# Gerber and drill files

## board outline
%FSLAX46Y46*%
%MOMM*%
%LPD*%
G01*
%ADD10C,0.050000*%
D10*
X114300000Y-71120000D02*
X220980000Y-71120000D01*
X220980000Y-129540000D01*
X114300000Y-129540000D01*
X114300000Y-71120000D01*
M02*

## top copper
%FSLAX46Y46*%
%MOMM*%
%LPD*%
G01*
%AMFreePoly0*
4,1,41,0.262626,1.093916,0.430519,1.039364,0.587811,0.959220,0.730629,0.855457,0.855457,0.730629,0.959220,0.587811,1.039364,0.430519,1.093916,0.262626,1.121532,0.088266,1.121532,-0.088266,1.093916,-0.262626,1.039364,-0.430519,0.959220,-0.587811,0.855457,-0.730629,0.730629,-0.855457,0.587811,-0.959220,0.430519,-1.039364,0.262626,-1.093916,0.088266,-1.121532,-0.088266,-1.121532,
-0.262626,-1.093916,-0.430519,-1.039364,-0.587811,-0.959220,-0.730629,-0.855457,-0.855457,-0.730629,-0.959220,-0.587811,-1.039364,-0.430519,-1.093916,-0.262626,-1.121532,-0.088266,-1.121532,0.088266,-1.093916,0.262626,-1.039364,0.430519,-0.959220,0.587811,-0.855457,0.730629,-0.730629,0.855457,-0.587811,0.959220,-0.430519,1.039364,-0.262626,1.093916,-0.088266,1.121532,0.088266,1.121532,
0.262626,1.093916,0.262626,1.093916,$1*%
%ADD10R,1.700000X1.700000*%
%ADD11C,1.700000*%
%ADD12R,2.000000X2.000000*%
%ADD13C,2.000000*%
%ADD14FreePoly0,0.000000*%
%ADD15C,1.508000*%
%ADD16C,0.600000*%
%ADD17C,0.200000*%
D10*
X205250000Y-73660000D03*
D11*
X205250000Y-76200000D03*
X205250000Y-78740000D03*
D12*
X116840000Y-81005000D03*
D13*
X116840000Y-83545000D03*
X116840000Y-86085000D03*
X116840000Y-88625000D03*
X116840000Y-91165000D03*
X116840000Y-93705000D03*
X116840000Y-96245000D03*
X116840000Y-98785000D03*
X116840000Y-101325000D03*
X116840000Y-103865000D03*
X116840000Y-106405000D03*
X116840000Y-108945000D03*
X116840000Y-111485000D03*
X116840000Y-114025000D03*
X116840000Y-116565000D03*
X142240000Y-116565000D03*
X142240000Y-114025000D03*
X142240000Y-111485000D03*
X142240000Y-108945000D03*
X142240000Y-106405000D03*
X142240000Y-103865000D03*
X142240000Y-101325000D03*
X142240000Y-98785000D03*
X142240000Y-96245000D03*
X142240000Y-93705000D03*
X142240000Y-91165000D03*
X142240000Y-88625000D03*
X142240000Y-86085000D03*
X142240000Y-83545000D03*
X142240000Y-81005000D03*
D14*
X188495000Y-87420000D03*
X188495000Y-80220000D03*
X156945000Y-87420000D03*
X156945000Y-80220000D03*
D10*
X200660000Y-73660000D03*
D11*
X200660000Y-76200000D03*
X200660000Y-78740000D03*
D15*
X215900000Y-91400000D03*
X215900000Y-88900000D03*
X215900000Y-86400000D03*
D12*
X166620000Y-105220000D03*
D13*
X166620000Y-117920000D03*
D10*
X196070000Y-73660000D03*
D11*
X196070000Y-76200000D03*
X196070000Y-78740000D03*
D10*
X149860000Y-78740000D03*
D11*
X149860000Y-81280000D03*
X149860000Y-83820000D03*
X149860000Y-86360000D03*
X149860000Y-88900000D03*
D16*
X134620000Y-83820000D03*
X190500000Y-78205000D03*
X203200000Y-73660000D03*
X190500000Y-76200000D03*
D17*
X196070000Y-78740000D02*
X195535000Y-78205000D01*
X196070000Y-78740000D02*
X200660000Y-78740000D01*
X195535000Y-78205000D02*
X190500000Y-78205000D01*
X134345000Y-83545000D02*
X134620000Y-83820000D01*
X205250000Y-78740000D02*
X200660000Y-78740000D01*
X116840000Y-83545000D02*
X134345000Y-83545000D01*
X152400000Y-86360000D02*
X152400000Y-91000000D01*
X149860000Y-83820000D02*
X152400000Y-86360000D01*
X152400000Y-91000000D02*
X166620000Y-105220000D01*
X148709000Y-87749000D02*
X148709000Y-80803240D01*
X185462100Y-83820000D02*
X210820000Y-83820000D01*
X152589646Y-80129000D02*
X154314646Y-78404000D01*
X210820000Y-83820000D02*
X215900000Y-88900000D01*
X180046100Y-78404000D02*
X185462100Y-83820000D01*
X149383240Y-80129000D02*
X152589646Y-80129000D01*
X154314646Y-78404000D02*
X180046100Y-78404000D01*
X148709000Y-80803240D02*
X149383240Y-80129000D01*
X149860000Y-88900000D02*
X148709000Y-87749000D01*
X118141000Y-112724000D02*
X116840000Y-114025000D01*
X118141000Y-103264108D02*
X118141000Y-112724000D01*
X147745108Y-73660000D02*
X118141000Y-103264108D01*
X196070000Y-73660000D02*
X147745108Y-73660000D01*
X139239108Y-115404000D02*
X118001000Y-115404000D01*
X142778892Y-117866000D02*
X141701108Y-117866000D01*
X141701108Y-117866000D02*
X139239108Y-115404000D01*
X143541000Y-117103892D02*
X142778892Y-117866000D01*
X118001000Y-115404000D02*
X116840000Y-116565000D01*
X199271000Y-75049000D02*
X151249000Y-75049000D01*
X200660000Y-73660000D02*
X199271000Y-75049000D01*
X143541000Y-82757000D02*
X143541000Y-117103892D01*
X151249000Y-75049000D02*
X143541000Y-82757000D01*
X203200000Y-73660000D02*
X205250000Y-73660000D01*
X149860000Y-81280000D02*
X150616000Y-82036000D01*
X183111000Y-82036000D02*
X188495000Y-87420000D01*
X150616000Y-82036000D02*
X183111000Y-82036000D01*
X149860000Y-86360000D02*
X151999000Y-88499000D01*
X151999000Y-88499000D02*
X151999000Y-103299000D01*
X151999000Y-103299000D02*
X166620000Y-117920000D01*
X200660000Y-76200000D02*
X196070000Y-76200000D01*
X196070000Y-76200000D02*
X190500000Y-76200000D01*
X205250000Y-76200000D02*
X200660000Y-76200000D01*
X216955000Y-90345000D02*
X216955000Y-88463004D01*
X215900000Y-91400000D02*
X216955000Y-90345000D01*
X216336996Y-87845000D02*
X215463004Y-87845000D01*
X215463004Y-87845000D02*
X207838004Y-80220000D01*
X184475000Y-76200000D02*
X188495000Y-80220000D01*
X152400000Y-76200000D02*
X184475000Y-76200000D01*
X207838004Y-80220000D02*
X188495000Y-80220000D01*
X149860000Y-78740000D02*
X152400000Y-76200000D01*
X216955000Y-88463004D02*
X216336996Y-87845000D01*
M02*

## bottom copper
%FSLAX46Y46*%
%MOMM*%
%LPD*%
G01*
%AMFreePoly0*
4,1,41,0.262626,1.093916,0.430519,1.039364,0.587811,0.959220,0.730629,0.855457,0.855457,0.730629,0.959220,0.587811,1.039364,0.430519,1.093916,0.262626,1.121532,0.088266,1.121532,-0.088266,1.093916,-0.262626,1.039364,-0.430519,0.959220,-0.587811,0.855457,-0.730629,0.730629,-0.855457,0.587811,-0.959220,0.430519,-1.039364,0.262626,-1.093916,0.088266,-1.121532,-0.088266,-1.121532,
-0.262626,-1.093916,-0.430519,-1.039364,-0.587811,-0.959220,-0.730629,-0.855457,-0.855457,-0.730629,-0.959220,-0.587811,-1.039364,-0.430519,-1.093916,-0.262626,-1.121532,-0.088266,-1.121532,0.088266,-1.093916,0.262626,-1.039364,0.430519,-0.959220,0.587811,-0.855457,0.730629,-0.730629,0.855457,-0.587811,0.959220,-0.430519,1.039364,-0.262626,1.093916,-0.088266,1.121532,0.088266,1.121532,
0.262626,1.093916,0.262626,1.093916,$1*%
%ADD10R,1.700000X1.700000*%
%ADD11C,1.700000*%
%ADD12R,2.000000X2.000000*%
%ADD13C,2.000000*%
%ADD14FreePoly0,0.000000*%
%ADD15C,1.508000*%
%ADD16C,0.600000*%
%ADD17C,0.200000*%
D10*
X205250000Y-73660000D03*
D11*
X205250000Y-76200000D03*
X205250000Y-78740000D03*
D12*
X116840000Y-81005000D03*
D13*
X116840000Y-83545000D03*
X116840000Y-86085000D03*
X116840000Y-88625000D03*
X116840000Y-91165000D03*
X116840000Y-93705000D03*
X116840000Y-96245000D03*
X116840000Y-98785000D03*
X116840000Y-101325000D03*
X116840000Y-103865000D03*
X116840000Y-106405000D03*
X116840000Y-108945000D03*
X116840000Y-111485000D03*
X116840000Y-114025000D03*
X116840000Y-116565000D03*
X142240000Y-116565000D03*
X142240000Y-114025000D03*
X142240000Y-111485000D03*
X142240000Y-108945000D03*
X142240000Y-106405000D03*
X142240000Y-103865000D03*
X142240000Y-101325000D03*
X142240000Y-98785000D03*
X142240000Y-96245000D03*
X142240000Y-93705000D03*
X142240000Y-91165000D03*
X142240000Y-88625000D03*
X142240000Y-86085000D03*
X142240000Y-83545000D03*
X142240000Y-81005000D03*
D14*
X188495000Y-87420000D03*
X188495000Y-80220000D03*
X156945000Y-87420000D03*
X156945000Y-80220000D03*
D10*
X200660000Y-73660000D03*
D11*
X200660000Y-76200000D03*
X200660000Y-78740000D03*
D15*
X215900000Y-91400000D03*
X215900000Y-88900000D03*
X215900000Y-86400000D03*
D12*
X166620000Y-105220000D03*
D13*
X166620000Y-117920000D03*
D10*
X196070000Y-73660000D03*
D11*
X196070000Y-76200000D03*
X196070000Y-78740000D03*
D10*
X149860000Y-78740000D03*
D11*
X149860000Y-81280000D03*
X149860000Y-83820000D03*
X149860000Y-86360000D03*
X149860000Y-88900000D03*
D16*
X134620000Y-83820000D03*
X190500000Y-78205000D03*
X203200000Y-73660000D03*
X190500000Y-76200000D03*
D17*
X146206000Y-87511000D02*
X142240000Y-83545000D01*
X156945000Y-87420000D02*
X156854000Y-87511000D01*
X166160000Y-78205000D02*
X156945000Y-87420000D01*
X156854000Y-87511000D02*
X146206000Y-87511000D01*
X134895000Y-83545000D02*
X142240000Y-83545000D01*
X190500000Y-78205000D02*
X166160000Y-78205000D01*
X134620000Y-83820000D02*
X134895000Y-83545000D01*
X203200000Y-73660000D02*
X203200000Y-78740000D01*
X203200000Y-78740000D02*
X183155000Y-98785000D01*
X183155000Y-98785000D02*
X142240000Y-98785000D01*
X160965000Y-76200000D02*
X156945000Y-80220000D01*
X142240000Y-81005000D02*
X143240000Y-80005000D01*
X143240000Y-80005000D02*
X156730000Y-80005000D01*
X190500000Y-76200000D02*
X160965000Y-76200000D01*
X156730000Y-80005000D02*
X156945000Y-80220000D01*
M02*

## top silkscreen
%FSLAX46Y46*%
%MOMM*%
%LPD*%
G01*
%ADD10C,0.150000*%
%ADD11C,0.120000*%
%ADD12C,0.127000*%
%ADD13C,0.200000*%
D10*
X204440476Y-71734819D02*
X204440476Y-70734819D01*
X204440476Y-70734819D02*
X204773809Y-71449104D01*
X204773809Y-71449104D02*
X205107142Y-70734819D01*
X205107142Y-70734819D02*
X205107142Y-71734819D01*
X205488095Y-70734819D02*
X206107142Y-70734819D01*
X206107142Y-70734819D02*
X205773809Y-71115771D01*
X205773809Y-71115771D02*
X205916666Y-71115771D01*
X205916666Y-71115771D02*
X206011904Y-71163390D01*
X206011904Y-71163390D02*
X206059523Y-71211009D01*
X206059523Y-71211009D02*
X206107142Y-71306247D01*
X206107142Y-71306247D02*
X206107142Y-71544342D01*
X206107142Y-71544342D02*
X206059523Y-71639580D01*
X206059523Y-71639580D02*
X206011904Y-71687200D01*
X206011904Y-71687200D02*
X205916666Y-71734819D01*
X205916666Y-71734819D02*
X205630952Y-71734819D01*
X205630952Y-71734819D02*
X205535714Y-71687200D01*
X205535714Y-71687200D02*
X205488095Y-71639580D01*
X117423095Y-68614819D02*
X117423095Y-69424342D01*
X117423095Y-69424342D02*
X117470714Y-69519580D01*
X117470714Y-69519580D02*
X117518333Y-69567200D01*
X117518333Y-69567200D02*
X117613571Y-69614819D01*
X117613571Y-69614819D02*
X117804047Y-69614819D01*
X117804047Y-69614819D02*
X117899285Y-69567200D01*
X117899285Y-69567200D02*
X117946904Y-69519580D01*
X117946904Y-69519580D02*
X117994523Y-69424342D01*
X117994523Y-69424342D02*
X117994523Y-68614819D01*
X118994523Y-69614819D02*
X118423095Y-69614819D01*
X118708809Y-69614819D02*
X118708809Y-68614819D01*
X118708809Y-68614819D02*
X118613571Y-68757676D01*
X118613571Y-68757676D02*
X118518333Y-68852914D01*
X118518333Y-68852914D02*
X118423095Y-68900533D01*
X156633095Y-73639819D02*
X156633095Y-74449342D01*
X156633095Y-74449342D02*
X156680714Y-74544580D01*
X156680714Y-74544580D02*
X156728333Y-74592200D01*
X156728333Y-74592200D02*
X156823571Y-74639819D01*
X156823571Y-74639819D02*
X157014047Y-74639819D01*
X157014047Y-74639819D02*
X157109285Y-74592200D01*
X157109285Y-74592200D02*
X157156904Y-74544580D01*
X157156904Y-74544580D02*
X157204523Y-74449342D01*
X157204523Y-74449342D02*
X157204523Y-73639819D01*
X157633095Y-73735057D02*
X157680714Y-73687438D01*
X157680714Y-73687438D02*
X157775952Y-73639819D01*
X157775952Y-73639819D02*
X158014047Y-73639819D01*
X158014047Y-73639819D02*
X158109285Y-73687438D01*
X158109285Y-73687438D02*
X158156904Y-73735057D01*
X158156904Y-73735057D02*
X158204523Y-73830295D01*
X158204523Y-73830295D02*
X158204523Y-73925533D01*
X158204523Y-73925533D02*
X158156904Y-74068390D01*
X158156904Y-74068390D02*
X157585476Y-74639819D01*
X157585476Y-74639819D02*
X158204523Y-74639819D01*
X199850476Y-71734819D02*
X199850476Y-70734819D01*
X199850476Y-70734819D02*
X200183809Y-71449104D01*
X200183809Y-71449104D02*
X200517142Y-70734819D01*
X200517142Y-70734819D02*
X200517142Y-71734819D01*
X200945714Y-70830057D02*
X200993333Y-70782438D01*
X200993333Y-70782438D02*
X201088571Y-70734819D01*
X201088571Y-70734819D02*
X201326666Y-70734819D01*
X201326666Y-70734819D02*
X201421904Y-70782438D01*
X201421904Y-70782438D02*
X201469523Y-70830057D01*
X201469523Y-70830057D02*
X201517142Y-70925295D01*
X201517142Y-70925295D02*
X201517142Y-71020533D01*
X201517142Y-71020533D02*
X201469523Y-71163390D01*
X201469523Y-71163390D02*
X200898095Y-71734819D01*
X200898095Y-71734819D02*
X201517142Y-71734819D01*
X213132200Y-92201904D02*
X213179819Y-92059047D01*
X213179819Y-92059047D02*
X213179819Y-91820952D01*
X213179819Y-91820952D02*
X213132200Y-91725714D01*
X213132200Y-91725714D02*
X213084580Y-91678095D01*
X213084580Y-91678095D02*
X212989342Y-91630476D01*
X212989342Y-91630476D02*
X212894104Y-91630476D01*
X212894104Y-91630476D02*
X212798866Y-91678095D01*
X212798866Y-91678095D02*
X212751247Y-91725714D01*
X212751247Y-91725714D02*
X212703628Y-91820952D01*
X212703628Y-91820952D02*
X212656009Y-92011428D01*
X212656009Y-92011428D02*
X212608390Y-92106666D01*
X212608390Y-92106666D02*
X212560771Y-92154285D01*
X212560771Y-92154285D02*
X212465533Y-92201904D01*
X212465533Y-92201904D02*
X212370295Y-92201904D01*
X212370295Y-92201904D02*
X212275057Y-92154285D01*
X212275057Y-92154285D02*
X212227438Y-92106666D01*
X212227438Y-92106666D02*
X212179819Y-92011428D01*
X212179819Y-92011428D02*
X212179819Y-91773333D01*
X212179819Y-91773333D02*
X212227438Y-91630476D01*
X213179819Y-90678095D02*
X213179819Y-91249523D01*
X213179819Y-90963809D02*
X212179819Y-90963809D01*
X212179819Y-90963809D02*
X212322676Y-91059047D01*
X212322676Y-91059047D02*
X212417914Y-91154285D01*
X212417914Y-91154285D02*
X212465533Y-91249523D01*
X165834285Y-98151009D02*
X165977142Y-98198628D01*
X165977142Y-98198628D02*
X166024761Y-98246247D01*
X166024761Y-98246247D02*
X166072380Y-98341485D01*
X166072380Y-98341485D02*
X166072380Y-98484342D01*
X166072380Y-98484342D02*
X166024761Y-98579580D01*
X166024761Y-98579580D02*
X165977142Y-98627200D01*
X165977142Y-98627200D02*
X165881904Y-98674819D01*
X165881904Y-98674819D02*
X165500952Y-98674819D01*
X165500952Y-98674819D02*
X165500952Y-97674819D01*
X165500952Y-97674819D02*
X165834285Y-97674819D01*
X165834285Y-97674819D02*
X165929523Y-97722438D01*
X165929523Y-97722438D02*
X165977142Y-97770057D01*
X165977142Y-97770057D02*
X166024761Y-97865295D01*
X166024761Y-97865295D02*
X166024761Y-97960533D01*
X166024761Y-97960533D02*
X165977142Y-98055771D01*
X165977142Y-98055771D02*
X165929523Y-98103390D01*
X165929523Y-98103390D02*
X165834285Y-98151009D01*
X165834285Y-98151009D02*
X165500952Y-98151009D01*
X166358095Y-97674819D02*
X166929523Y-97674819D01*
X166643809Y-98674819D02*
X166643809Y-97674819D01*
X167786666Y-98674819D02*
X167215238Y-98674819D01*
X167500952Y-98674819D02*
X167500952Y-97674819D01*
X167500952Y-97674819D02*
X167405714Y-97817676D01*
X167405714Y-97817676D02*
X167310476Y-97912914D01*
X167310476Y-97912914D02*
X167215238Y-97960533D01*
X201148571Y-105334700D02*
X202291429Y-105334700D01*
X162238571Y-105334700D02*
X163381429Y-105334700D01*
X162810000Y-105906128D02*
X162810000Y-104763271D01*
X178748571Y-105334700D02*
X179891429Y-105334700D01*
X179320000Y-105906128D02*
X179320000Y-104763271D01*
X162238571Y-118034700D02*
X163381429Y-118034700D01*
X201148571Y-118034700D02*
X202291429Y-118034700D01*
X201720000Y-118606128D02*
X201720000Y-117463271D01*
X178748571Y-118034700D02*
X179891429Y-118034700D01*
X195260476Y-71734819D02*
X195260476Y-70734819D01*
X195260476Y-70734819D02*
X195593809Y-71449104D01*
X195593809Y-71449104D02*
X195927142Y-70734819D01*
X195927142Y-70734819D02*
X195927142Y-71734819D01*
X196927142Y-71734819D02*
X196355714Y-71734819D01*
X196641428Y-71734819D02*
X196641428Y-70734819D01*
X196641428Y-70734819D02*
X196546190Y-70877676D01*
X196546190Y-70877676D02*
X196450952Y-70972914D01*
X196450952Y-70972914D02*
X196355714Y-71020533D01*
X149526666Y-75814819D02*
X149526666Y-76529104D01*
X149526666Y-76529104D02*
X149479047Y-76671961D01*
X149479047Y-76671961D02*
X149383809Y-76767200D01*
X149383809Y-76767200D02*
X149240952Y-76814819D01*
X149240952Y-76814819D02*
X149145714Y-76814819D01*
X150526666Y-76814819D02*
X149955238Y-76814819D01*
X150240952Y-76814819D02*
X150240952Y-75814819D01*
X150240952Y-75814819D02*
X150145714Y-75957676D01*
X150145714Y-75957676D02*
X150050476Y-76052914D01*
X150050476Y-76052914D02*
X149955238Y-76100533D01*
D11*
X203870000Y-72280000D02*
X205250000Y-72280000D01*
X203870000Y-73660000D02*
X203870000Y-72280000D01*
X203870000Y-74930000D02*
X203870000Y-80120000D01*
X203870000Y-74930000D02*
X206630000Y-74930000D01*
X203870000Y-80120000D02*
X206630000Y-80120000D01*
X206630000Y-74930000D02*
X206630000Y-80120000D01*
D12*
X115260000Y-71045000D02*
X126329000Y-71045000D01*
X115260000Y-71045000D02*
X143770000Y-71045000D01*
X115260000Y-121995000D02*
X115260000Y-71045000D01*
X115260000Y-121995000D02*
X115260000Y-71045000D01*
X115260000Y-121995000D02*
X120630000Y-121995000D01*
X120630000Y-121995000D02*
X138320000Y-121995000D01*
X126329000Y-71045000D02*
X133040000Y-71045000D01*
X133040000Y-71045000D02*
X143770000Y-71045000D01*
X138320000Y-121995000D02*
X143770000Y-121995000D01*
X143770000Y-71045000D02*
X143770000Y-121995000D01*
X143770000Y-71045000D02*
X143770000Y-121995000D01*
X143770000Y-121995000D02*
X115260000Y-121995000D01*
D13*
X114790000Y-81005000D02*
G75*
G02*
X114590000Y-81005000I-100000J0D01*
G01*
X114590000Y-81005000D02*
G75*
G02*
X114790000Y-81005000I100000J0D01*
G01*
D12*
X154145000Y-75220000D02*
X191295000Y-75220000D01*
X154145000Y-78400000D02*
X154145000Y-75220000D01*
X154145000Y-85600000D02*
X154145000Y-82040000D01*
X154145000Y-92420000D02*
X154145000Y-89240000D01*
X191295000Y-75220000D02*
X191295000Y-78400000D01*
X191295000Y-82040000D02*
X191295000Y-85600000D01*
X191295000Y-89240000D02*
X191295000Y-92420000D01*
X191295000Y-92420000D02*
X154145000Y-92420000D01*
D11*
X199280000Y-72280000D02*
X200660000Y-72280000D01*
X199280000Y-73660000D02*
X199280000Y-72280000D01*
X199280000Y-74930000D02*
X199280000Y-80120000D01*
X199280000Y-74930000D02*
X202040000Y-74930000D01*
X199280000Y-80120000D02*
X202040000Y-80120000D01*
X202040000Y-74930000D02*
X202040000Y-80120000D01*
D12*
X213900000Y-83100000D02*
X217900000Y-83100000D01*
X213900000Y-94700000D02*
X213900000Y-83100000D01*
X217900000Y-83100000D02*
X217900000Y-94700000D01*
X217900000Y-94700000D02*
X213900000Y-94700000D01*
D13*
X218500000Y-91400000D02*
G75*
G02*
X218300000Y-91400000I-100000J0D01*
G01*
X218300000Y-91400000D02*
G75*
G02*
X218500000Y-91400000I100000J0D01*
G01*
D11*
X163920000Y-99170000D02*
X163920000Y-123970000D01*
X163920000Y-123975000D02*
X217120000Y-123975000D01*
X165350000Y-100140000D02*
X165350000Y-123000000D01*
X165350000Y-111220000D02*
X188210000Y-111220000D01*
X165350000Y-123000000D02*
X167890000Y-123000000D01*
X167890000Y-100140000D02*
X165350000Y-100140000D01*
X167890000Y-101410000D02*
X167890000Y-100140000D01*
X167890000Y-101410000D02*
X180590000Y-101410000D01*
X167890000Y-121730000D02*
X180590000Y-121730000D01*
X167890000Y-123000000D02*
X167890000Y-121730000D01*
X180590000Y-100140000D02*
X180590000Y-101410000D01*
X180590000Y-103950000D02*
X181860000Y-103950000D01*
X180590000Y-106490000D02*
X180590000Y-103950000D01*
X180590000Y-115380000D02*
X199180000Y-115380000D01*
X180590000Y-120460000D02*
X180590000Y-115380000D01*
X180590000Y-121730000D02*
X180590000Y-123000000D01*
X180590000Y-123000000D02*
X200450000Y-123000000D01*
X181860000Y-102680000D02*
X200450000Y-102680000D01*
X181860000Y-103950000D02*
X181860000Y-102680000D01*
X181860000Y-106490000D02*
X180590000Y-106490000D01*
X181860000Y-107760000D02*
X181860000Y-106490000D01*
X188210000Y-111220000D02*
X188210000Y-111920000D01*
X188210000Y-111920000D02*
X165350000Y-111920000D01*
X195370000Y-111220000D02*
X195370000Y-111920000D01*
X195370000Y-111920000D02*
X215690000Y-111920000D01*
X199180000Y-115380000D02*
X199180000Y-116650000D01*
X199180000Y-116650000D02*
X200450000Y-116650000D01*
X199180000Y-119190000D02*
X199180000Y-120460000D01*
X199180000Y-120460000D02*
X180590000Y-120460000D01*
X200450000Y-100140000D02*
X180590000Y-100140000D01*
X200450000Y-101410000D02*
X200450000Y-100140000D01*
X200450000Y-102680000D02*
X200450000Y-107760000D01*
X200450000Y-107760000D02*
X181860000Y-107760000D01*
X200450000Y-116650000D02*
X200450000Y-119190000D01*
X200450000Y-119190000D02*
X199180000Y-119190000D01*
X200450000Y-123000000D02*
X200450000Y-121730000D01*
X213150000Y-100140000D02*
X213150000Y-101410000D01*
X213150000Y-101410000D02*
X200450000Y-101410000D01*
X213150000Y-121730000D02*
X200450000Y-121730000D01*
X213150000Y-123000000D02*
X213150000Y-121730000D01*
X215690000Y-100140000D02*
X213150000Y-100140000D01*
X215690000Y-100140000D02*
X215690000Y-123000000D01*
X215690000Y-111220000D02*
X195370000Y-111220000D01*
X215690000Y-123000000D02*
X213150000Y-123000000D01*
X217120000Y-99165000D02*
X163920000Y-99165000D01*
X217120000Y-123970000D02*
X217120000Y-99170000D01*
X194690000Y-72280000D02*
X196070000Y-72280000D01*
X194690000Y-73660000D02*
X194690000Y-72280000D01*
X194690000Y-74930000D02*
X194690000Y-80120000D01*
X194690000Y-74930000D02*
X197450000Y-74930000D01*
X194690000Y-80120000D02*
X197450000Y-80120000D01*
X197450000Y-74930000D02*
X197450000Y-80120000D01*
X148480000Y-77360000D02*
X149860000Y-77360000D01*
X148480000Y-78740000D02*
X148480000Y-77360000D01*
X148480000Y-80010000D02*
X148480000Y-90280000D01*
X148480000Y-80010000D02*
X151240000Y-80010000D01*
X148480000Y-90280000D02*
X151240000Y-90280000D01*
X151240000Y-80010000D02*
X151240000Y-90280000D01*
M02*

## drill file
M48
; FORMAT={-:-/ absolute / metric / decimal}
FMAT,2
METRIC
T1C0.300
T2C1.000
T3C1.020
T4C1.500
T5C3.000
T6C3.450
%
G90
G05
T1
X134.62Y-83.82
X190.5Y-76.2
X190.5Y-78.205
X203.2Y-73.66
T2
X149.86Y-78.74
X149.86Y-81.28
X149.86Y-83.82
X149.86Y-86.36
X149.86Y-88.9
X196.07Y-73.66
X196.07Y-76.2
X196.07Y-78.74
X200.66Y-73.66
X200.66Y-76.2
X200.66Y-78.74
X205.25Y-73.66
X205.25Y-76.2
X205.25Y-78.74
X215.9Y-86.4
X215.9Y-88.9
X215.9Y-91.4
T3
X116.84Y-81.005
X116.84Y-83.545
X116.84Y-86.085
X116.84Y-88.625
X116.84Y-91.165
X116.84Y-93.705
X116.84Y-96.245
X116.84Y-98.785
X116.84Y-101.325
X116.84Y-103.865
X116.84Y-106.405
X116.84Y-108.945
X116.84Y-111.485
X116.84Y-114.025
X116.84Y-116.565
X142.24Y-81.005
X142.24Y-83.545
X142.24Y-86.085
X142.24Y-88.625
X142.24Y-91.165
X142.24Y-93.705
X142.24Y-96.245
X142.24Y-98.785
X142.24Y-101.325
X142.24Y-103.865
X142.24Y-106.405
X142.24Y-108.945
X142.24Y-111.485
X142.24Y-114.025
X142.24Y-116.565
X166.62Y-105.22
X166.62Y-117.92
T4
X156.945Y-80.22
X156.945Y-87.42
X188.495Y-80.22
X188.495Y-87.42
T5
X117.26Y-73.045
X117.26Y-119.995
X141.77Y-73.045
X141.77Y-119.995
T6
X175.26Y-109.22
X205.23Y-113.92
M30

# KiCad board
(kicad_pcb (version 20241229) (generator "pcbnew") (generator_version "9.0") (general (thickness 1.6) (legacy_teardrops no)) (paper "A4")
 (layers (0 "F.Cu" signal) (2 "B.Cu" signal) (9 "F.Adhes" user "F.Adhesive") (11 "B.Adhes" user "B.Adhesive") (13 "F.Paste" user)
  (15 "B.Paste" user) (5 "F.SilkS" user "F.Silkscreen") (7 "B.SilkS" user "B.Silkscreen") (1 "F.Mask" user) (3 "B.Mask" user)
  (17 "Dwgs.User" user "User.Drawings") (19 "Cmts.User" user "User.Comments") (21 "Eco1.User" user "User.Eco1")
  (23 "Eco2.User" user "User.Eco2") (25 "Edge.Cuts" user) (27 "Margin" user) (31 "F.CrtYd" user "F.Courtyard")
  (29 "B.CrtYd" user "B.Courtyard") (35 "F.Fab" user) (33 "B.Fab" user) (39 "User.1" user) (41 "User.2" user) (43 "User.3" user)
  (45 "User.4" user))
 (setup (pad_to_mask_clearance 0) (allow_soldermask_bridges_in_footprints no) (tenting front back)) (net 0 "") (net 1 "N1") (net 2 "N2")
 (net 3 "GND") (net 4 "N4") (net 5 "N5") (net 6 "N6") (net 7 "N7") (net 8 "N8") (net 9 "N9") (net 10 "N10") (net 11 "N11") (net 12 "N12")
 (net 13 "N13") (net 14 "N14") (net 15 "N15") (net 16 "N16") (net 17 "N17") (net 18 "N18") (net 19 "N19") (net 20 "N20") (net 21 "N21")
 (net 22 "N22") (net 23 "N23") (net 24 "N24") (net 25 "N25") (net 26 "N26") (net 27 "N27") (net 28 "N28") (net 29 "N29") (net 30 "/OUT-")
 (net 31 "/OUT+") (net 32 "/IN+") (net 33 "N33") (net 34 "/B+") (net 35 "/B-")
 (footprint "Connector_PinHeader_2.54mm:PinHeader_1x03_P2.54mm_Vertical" (layer "F.Cu") (at 205.25 73.66)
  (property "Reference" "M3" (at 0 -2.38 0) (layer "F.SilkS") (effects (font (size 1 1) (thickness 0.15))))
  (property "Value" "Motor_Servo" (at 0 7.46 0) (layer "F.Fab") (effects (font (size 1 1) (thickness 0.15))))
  (fp_line (start -1.38 -1.38) (end 0 -1.38) (stroke (width 0.12) (type solid)) (layer "F.SilkS"))
  (fp_line (start -1.38 0) (end -1.38 -1.38) (stroke (width 0.12) (type solid)) (layer "F.SilkS"))
  (fp_line (start -1.38 1.27) (end -1.38 6.46) (stroke (width 0.12) (type solid)) (layer "F.SilkS"))
  (fp_line (start -1.38 1.27) (end 1.38 1.27) (stroke (width 0.12) (type solid)) (layer "F.SilkS"))
  (fp_line (start -1.38 6.46) (end 1.38 6.46) (stroke (width 0.12) (type solid)) (layer "F.SilkS"))
  (fp_line (start 1.38 1.27) (end 1.38 6.46) (stroke (width 0.12) (type solid)) (layer "F.SilkS"))
  (pad "1" thru_hole rect (at 0 0) (size 1.7 1.7) (drill 1) (layers "*.Cu" "*.Mask") (remove_unused_layers no) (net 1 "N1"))
  (pad "2" thru_hole circle (at 0 2.54) (size 1.7 1.7) (drill 1) (layers "*.Cu" "*.Mask") (remove_unused_layers no) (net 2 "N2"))
  (pad "3" thru_hole circle (at 0 5.08) (size 1.7 1.7) (drill 1) (layers "*.Cu" "*.Mask") (remove_unused_layers no) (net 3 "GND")))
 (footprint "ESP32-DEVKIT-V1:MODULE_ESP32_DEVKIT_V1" (layer "F.Cu") (at 129.54 96.52)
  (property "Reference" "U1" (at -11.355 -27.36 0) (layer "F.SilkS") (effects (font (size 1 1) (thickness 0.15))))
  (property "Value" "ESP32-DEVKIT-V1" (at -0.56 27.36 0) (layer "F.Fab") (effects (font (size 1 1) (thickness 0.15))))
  (fp_line (start -14.28 -25.475) (end -3.211 -25.475) (stroke (width 0.127) (type solid)) (layer "F.SilkS"))
  (fp_line (start -14.28 -25.475) (end 14.23 -25.475) (stroke (width 0.127) (type solid)) (layer "F.SilkS"))
  (fp_line (start -14.28 25.475) (end -14.28 -25.475) (stroke (width 0.127) (type solid)) (layer "F.SilkS"))
  (fp_line (start -14.28 25.475) (end -14.28 -25.475) (stroke (width 0.127) (type solid)) (layer "F.SilkS"))
  (fp_line (start -14.28 25.475) (end -8.91 25.475) (stroke (width 0.127) (type solid)) (layer "F.SilkS"))
  (fp_line (start -8.91 25.475) (end 8.78 25.475) (stroke (width 0.127) (type solid)) (layer "F.SilkS"))
  (fp_line (start -3.211 -25.475) (end 3.5 -25.475) (stroke (width 0.127) (type solid)) (layer "F.SilkS"))
  (fp_line (start 3.5 -25.475) (end 14.23 -25.475) (stroke (width 0.127) (type solid)) (layer "F.SilkS"))
  (fp_line (start 8.78 25.475) (end 14.23 25.475) (stroke (width 0.127) (type solid)) (layer "F.SilkS"))
  (fp_line (start 14.23 -25.475) (end 14.23 25.475) (stroke (width 0.127) (type solid)) (layer "F.SilkS"))
  (fp_line (start 14.23 -25.475) (end 14.23 25.475) (stroke (width 0.127) (type solid)) (layer "F.SilkS"))
  (fp_line (start 14.23 25.475) (end -14.28 25.475) (stroke (width 0.127) (type solid)) (layer "F.SilkS"))
  (fp_circle (center -14.85 -15.515) (end -14.75 -15.515) (stroke (width 0.2) (type solid)) (fill no) (layer "F.SilkS"))
  (pad "" np_thru_hole circle (at -12.28 -23.475) (size 3 3) (drill 3) (layers "*.Cu" "*.Mask"))
  (pad "" np_thru_hole circle (at -12.28 23.475) (size 3 3) (drill 3) (layers "*.Cu" "*.Mask"))
  (pad "" np_thru_hole circle (at 12.23 -23.475) (size 3 3) (drill 3) (layers "*.Cu" "*.Mask"))
  (pad "" np_thru_hole circle (at 12.23 23.475) (size 3 3) (drill 3) (layers "*.Cu" "*.Mask"))
  (pad "1" thru_hole rect (at -12.7 -15.515) (size 2 2) (drill 1.02) (layers "*.Cu" "*.Mask") (remove_unused_layers no) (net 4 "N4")
   (solder_mask_margin 0.102))
  (pad "2" thru_hole circle (at -12.7 -12.975) (size 2 2) (drill 1.02) (layers "*.Cu" "*.Mask") (remove_unused_layers no) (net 3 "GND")
   (solder_mask_margin 0.102))
  (pad "3" thru_hole circle (at -12.7 -10.435) (size 2 2) (drill 1.02) (layers "*.Cu" "*.Mask") (remove_unused_layers no) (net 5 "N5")
   (solder_mask_margin 0.102))
  (pad "4" thru_hole circle (at -12.7 -7.895) (size 2 2) (drill 1.02) (layers "*.Cu" "*.Mask") (remove_unused_layers no) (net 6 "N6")
   (solder_mask_margin 0.102))
  (pad "5" thru_hole circle (at -12.7 -5.355) (size 2 2) (drill 1.02) (layers "*.Cu" "*.Mask") (remove_unused_layers no) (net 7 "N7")
   (solder_mask_margin 0.102))
  (pad "6" thru_hole circle (at -12.7 -2.815) (size 2 2) (drill 1.02) (layers "*.Cu" "*.Mask") (remove_unused_layers no) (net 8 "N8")
   (solder_mask_margin 0.102))
  (pad "7" thru_hole circle (at -12.7 -0.275) (size 2 2) (drill 1.02) (layers "*.Cu" "*.Mask") (remove_unused_layers no) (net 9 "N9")
   (solder_mask_margin 0.102))
  (pad "8" thru_hole circle (at -12.7 2.265) (size 2 2) (drill 1.02) (layers "*.Cu" "*.Mask") (remove_unused_layers no) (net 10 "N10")
   (solder_mask_margin 0.102))
  (pad "9" thru_hole circle (at -12.7 4.805) (size 2 2) (drill 1.02) (layers "*.Cu" "*.Mask") (remove_unused_layers no) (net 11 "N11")
   (solder_mask_margin 0.102))
  (pad "10" thru_hole circle (at -12.7 7.345) (size 2 2) (drill 1.02) (layers "*.Cu" "*.Mask") (remove_unused_layers no) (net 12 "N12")
   (solder_mask_margin 0.102))
  (pad "11" thru_hole circle (at -12.7 9.885) (size 2 2) (drill 1.02) (layers "*.Cu" "*.Mask") (remove_unused_layers no) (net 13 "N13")
   (solder_mask_margin 0.102))
  (pad "12" thru_hole circle (at -12.7 12.425) (size 2 2) (drill 1.02) (layers "*.Cu" "*.Mask") (remove_unused_layers no) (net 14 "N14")
   (solder_mask_margin 0.102))
  (pad "13" thru_hole circle (at -12.7 14.965) (size 2 2) (drill 1.02) (layers "*.Cu" "*.Mask") (remove_unused_layers no) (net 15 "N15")
   (solder_mask_margin 0.102))
  (pad "14" thru_hole circle (at -12.7 17.505) (size 2 2) (drill 1.02) (layers "*.Cu" "*.Mask") (remove_unused_layers no) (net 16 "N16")
   (solder_mask_margin 0.102))
  (pad "15" thru_hole circle (at -12.7 20.045) (size 2 2) (drill 1.02) (layers "*.Cu" "*.Mask") (remove_unused_layers no) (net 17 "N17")
   (solder_mask_margin 0.102))
  (pad "16" thru_hole circle (at 12.7 20.045) (size 2 2) (drill 1.02) (layers "*.Cu" "*.Mask") (remove_unused_layers no) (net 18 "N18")
   (solder_mask_margin 0.102))
  (pad "17" thru_hole circle (at 12.7 17.505) (size 2 2) (drill 1.02) (layers "*.Cu" "*.Mask") (remove_unused_layers no) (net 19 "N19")
   (solder_mask_margin 0.102))
  (pad "18" thru_hole circle (at 12.7 14.965) (size 2 2) (drill 1.02) (layers "*.Cu" "*.Mask") (remove_unused_layers no) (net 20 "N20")
   (solder_mask_margin 0.102))
  (pad "19" thru_hole circle (at 12.7 12.425) (size 2 2) (drill 1.02) (layers "*.Cu" "*.Mask") (remove_unused_layers no) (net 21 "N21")
   (solder_mask_margin 0.102))
  (pad "20" thru_hole circle (at 12.7 9.885) (size 2 2) (drill 1.02) (layers "*.Cu" "*.Mask") (remove_unused_layers no) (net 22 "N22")
   (solder_mask_margin 0.102))
  (pad "21" thru_hole circle (at 12.7 7.345) (size 2 2) (drill 1.02) (layers "*.Cu" "*.Mask") (remove_unused_layers no) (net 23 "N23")
   (solder_mask_margin 0.102))
  (pad "22" thru_hole circle (at 12.7 4.805) (size 2 2) (drill 1.02) (layers "*.Cu" "*.Mask") (remove_unused_layers no) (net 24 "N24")
   (solder_mask_margin 0.102))
  (pad "23" thru_hole circle (at 12.7 2.265) (size 2 2) (drill 1.02) (layers "*.Cu" "*.Mask") (remove_unused_layers no) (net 1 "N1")
   (solder_mask_margin 0.102))
  (pad "24" thru_hole circle (at 12.7 -0.275) (size 2 2) (drill 1.02) (layers "*.Cu" "*.Mask") (remove_unused_layers no) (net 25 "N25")
   (solder_mask_margin 0.102))
  (pad "25" thru_hole circle (at 12.7 -2.815) (size 2 2) (drill 1.02) (layers "*.Cu" "*.Mask") (remove_unused_layers no) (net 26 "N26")
   (solder_mask_margin 0.102))
  (pad "26" thru_hole circle (at 12.7 -5.355) (size 2 2) (drill 1.02) (layers "*.Cu" "*.Mask") (remove_unused_layers no) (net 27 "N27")
   (solder_mask_margin 0.102))
  (pad "27" thru_hole circle (at 12.7 -7.895) (size 2 2) (drill 1.02) (layers "*.Cu" "*.Mask") (remove_unused_layers no) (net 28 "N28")
   (solder_mask_margin 0.102))
  (pad "28" thru_hole circle (at 12.7 -10.435) (size 2 2) (drill 1.02) (layers "*.Cu" "*.Mask") (remove_unused_layers no) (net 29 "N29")
   (solder_mask_margin 0.102))
  (pad "29" thru_hole circle (at 12.7 -12.975) (size 2 2) (drill 1.02) (layers "*.Cu" "*.Mask") (remove_unused_layers no) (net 3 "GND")
   (solder_mask_margin 0.102))
  (pad "30" thru_hole circle (at 12.7 -15.515) (size 2 2) (drill 1.02) (layers "*.Cu" "*.Mask") (remove_unused_layers no) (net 2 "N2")
   (solder_mask_margin 0.102))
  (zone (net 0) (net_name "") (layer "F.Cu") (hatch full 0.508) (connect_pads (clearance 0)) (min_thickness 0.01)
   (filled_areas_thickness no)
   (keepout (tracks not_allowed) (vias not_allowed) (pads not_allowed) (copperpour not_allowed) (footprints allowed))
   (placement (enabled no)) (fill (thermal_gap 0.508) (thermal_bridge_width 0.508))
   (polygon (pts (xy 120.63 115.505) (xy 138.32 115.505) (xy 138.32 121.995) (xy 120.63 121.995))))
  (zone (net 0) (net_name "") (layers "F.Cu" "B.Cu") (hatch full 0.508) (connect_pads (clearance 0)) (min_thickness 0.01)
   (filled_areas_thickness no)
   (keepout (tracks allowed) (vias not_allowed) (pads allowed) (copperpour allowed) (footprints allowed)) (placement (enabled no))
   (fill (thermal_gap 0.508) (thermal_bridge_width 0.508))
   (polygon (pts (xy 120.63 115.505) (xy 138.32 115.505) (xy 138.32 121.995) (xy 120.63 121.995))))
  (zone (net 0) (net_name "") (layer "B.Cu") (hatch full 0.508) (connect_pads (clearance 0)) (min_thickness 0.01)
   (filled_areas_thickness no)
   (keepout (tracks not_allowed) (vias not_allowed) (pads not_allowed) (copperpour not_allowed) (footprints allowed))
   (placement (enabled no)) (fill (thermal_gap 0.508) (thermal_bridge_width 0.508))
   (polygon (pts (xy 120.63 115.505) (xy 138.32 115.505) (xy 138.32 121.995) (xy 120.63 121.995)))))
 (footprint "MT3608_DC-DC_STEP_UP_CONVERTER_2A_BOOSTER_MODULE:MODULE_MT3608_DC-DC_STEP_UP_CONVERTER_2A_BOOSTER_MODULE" (layer "F.Cu")
  (at 172.72 83.82)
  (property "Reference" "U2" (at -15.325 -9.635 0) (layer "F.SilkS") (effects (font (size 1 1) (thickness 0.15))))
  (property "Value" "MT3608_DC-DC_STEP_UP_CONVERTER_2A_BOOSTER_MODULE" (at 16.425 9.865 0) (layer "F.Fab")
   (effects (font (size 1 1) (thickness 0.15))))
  (fp_line (start -18.575 -8.6) (end 18.575 -8.6) (stroke (width 0.127) (type solid)) (layer "F.SilkS"))
  (fp_line (start -18.575 -5.42) (end -18.575 -8.6) (stroke (width 0.127) (type solid)) (layer "F.SilkS"))
  (fp_line (start -18.575 1.78) (end -18.575 -1.78) (stroke (width 0.127) (type solid)) (layer "F.SilkS"))
  (fp_line (start -18.575 8.6) (end -18.575 5.42) (stroke (width 0.127) (type solid)) (layer "F.SilkS"))
  (fp_line (start 18.575 -8.6) (end 18.575 -5.42) (stroke (width 0.127) (type solid)) (layer "F.SilkS"))
  (fp_line (start 18.575 -1.78) (end 18.575 1.78) (stroke (width 0.127) (type solid)) (layer "F.SilkS"))
  (fp_line (start 18.575 5.42) (end 18.575 8.6) (stroke (width 0.127) (type solid)) (layer "F.SilkS"))
  (fp_line (start 18.575 8.6) (end -18.575 8.6) (stroke (width 0.127) (type solid)) (layer "F.SilkS"))
  (pad "VIN_N" thru_hole custom (at 15.775 3.6) (size 2.25 2.25) (drill 1.5) (layers "*.Cu") (remove_unused_layers no) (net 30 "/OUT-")
   (thermal_bridge_angle 90) (options (clearance outline) (anchor circle)) (primitives))
  (pad "VIN_P" thru_hole custom (at 15.775 -3.6) (size 2.25 2.25) (drill 1.5) (layers "*.Cu") (remove_unused_layers no) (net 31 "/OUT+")
   (thermal_bridge_angle 90) (options (clearance outline) (anchor circle)) (primitives))
  (pad "VOUT_N" thru_hole custom (at -15.775 3.6) (size 2.25 2.25) (drill 1.5) (layers "*.Cu") (remove_unused_layers no) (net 3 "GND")
   (thermal_bridge_angle 90) (options (clearance outline) (anchor circle)) (primitives))
  (pad "VOUT_P" thru_hole custom (at -15.775 -3.6) (size 2.25 2.25) (drill 1.5) (layers "*.Cu") (remove_unused_layers no) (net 2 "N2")
   (thermal_bridge_angle 90) (options (clearance outline) (anchor circle)) (primitives)))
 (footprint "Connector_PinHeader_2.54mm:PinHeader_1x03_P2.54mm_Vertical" (layer "F.Cu") (at 200.66 73.66)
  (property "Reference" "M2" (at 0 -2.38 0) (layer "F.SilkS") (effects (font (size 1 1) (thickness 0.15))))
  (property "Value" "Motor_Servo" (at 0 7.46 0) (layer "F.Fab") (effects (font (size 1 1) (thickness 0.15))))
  (fp_line (start -1.38 -1.38) (end 0 -1.38) (stroke (width 0.12) (type solid)) (layer "F.SilkS"))
  (fp_line (start -1.38 0) (end -1.38 -1.38) (stroke (width 0.12) (type solid)) (layer "F.SilkS"))
  (fp_line (start -1.38 1.27) (end -1.38 6.46) (stroke (width 0.12) (type solid)) (layer "F.SilkS"))
  (fp_line (start -1.38 1.27) (end 1.38 1.27) (stroke (width 0.12) (type solid)) (layer "F.SilkS"))
  (fp_line (start -1.38 6.46) (end 1.38 6.46) (stroke (width 0.12) (type solid)) (layer "F.SilkS"))
  (fp_line (start 1.38 1.27) (end 1.38 6.46) (stroke (width 0.12) (type solid)) (layer "F.SilkS"))
  (pad "1" thru_hole rect (at 0 0) (size 1.7 1.7) (drill 1) (layers "*.Cu" "*.Mask") (remove_unused_layers no) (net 17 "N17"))
  (pad "2" thru_hole circle (at 0 2.54) (size 1.7 1.7) (drill 1) (layers "*.Cu" "*.Mask") (remove_unused_layers no) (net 2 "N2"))
  (pad "3" thru_hole circle (at 0 5.08) (size 1.7 1.7) (drill 1) (layers "*.Cu" "*.Mask") (remove_unused_layers no) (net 3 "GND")))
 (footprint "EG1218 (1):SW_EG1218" (layer "F.Cu") (at 215.9 88.9 90)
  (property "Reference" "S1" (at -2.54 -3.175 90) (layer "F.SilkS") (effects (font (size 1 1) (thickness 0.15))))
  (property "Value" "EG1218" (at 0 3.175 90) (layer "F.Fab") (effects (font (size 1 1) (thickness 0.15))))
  (fp_line (start 5.8 -2) (end 5.8 2) (stroke (width 0.127) (type solid)) (layer "F.SilkS"))
  (fp_line (start -5.8 -2) (end 5.8 -2) (stroke (width 0.127) (type solid)) (layer "F.SilkS"))
  (fp_line (start 5.8 2) (end -5.8 2) (stroke (width 0.127) (type solid)) (layer "F.SilkS"))
  (fp_line (start -5.8 2) (end -5.8 -2) (stroke (width 0.127) (type solid)) (layer "F.SilkS"))
  (fp_circle (center -2.5 2.5) (end -2.4 2.5) (stroke (width 0.2) (type solid)) (fill no) (layer "F.SilkS"))
  (pad "1" thru_hole circle (at -2.5 0 90) (size 1.508 1.508) (drill 1) (layers "*.Cu" "*.Mask") (remove_unused_layers no) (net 31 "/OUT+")
   (solder_mask_margin 0.102))
  (pad "2" thru_hole circle (at 0 0 90) (size 1.508 1.508) (drill 1) (layers "*.Cu" "*.Mask") (remove_unused_layers no) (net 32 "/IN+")
   (solder_mask_margin 0.102))
  (pad "3" thru_hole circle (at 2.5 0 90) (size 1.508 1.508) (drill 1) (layers "*.Cu" "*.Mask") (remove_unused_layers no) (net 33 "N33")
   (solder_mask_margin 0.102)))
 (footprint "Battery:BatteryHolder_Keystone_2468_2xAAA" (layer "F.Cu") (at 166.62 105.22)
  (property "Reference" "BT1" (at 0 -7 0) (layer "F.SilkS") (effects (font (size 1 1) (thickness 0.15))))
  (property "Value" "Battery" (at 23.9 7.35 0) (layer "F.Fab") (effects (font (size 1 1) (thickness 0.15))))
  (fp_line (start -2.7 -6.05) (end -2.7 18.75) (stroke (width 0.12) (type solid)) (layer "F.SilkS"))
  (fp_line (start -2.7 18.755) (end 50.5 18.755) (stroke (width 0.12) (type solid)) (layer "F.SilkS"))
  (fp_line (start -1.27 -5.08) (end -1.27 17.78) (stroke (width 0.12) (type solid)) (layer "F.SilkS"))
  (fp_line (start -1.27 6) (end 21.59 6) (stroke (width 0.12) (type solid)) (layer "F.SilkS"))
  (fp_line (start -1.27 17.78) (end 1.27 17.78) (stroke (width 0.12) (type solid)) (layer "F.SilkS"))
  (fp_line (start 1.27 -5.08) (end -1.27 -5.08) (stroke (width 0.12) (type solid)) (layer "F.SilkS"))
  (fp_line (start 1.27 -3.81) (end 1.27 -5.08) (stroke (width 0.12) (type solid)) (layer "F.SilkS"))
  (fp_line (start 1.27 -3.81) (end 13.97 -3.81) (stroke (width 0.12) (type solid)) (layer "F.SilkS"))
  (fp_line (start 1.27 16.51) (end 13.97 16.51) (stroke (width 0.12) (type solid)) (layer "F.SilkS"))
  (fp_line (start 1.27 17.78) (end 1.27 16.51) (stroke (width 0.12) (type solid)) (layer "F.SilkS"))
  (fp_line (start 13.97 -5.08) (end 13.97 -3.81) (stroke (width 0.12) (type solid)) (layer "F.SilkS"))
  (fp_line (start 13.97 -1.27) (end 15.24 -1.27) (stroke (width 0.12) (type solid)) (layer "F.SilkS"))
  (fp_line (start 13.97 1.27) (end 13.97 -1.27) (stroke (width 0.12) (type solid)) (layer "F.SilkS"))
  (fp_line (start 13.97 10.16) (end 32.56 10.16) (stroke (width 0.12) (type solid)) (layer "F.SilkS"))
  (fp_line (start 13.97 15.24) (end 13.97 10.16) (stroke (width 0.12) (type solid)) (layer "F.SilkS"))
  (fp_line (start 13.97 16.51) (end 13.97 17.78) (stroke (width 0.12) (type solid)) (layer "F.SilkS"))
  (fp_line (start 13.97 17.78) (end 33.83 17.78) (stroke (width 0.12) (type solid)) (layer "F.SilkS"))
  (fp_line (start 15.24 -2.54) (end 33.83 -2.54) (stroke (width 0.12) (type solid)) (layer "F.SilkS"))
  (fp_line (start 15.24 -1.27) (end 15.24 -2.54) (stroke (width 0.12) (type solid)) (layer "F.SilkS"))
  (fp_line (start 15.24 1.27) (end 13.97 1.27) (stroke (width 0.12) (type solid)) (layer "F.SilkS"))
  (fp_line (start 15.24 2.54) (end 15.24 1.27) (stroke (width 0.12) (type solid)) (layer "F.SilkS"))
  (fp_line (start 21.59 6) (end 21.59 6.7) (stroke (width 0.12) (type solid)) (layer "F.SilkS"))
  (fp_line (start 21.59 6.7) (end -1.27 6.7) (stroke (width 0.12) (type solid)) (layer "F.SilkS"))
  (fp_line (start 28.75 6) (end 28.75 6.7) (stroke (width 0.12) (type solid)) (layer "F.SilkS"))
  (fp_line (start 28.75 6.7) (end 49.07 6.7) (stroke (width 0.12) (type solid)) (layer "F.SilkS"))
  (fp_line (start 32.56 10.16) (end 32.56 11.43) (stroke (width 0.12) (type solid)) (layer "F.SilkS"))
  (fp_line (start 32.56 11.43) (end 33.83 11.43) (stroke (width 0.12) (type solid)) (layer "F.SilkS"))
  (fp_line (start 32.56 13.97) (end 32.56 15.24) (stroke (width 0.12) (type solid)) (layer "F.SilkS"))
  (fp_line (start 32.56 15.24) (end 13.97 15.24) (stroke (width 0.12) (type solid)) (layer "F.SilkS"))
  (fp_line (start 33.83 -5.08) (end 13.97 -5.08) (stroke (width 0.12) (type solid)) (layer "F.SilkS"))
  (fp_line (start 33.83 -3.81) (end 33.83 -5.08) (stroke (width 0.12) (type solid)) (layer "F.SilkS"))
  (fp_line (start 33.83 -2.54) (end 33.83 2.54) (stroke (width 0.12) (type solid)) (layer "F.SilkS"))
  (fp_line (start 33.83 2.54) (end 15.24 2.54) (stroke (width 0.12) (type solid)) (layer "F.SilkS"))
  (fp_line (start 33.83 11.43) (end 33.83 13.97) (stroke (width 0.12) (type solid)) (layer "F.SilkS"))
  (fp_line (start 33.83 13.97) (end 32.56 13.97) (stroke (width 0.12) (type solid)) (layer "F.SilkS"))
  (fp_line (start 33.83 17.78) (end 33.83 16.51) (stroke (width 0.12) (type solid)) (layer "F.SilkS"))
  (fp_line (start 46.53 -5.08) (end 46.53 -3.81) (stroke (width 0.12) (type solid)) (layer "F.SilkS"))
  (fp_line (start 46.53 -3.81) (end 33.83 -3.81) (stroke (width 0.12) (type solid)) (layer "F.SilkS"))
  (fp_line (start 46.53 16.51) (end 33.83 16.51) (stroke (width 0.12) (type solid)) (layer "F.SilkS"))
  (fp_line (start 46.53 17.78) (end 46.53 16.51) (stroke (width 0.12) (type solid)) (layer "F.SilkS"))
  (fp_line (start 49.07 -5.08) (end 46.53 -5.08) (stroke (width 0.12) (type solid)) (layer "F.SilkS"))
  (fp_line (start 49.07 -5.08) (end 49.07 17.78) (stroke (width 0.12) (type solid)) (layer "F.SilkS"))
  (fp_line (start 49.07 6) (end 28.75 6) (stroke (width 0.12) (type solid)) (layer "F.SilkS"))
  (fp_line (start 49.07 17.78) (end 46.53 17.78) (stroke (width 0.12) (type solid)) (layer "F.SilkS"))
  (fp_line (start 50.5 -6.055) (end -2.7 -6.055) (stroke (width 0.12) (type solid)) (layer "F.SilkS"))
  (fp_line (start 50.5 18.75) (end 50.5 -6.05) (stroke (width 0.12) (type solid)) (layer "F.SilkS"))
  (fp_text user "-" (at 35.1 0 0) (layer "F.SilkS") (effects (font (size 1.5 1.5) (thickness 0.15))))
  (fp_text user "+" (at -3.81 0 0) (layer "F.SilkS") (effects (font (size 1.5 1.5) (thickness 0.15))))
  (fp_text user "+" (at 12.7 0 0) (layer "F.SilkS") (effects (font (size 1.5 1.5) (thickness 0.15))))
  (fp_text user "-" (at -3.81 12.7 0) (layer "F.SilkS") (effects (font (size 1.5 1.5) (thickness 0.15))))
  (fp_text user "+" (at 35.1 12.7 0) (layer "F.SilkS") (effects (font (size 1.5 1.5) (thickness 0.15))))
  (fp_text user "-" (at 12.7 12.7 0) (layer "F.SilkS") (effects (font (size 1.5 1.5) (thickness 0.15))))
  (pad "" np_thru_hole circle (at 8.64 4) (size 3.45 3.45) (drill 3.45) (layers "*.Cu"))
  (pad "" np_thru_hole circle (at 38.61 8.7) (size 3.45 3.45) (drill 3.45) (layers "*.Cu" "*.Mask"))
  (pad "1" thru_hole rect (at 0 0) (size 2 2) (drill 1.02) (layers "*.Cu" "*.Mask") (remove_unused_layers no) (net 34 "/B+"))
  (pad "2" thru_hole circle (at 0 12.7) (size 2 2) (drill 1.02) (layers "*.Cu" "*.Mask") (remove_unused_layers no) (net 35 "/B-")))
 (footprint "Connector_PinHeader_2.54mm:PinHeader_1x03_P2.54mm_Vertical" (layer "F.Cu") (at 196.07 73.66)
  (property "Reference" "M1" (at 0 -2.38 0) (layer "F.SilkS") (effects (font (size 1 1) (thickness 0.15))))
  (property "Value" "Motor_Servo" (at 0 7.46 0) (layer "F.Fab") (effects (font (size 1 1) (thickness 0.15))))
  (fp_line (start -1.38 -1.38) (end 0 -1.38) (stroke (width 0.12) (type solid)) (layer "F.SilkS"))
  (fp_line (start -1.38 0) (end -1.38 -1.38) (stroke (width 0.12) (type solid)) (layer "F.SilkS"))
  (fp_line (start -1.38 1.27) (end -1.38 6.46) (stroke (width 0.12) (type solid)) (layer "F.SilkS"))
  (fp_line (start -1.38 1.27) (end 1.38 1.27) (stroke (width 0.12) (type solid)) (layer "F.SilkS"))
  (fp_line (start -1.38 6.46) (end 1.38 6.46) (stroke (width 0.12) (type solid)) (layer "F.SilkS"))
  (fp_line (start 1.38 1.27) (end 1.38 6.46) (stroke (width 0.12) (type solid)) (layer "F.SilkS"))
  (pad "1" thru_hole rect (at 0 0) (size 1.7 1.7) (drill 1) (layers "*.Cu" "*.Mask") (remove_unused_layers no) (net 16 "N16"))
  (pad "2" thru_hole circle (at 0 2.54) (size 1.7 1.7) (drill 1) (layers "*.Cu" "*.Mask") (remove_unused_layers no) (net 2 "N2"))
  (pad "3" thru_hole circle (at 0 5.08) (size 1.7 1.7) (drill 1) (layers "*.Cu" "*.Mask") (remove_unused_layers no) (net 3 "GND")))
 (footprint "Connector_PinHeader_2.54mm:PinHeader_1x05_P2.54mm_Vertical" (layer "F.Cu") (at 149.86 78.74)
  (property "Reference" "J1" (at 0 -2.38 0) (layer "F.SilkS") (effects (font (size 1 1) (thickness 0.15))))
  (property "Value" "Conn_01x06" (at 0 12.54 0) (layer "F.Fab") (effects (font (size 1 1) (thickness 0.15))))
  (fp_line (start -1.38 -1.38) (end 0 -1.38) (stroke (width 0.12) (type solid)) (layer "F.SilkS"))
  (fp_line (start -1.38 0) (end -1.38 -1.38) (stroke (width 0.12) (type solid)) (layer "F.SilkS"))
  (fp_line (start -1.38 1.27) (end -1.38 11.54) (stroke (width 0.12) (type solid)) (layer "F.SilkS"))
  (fp_line (start -1.38 1.27) (end 1.38 1.27) (stroke (width 0.12) (type solid)) (layer "F.SilkS"))
  (fp_line (start -1.38 11.54) (end 1.38 11.54) (stroke (width 0.12) (type solid)) (layer "F.SilkS"))
  (fp_line (start 1.38 1.27) (end 1.38 11.54) (stroke (width 0.12) (type solid)) (layer "F.SilkS"))
  (pad "1" thru_hole rect (at 0 0) (size 1.7 1.7) (drill 1) (layers "*.Cu" "*.Mask") (remove_unused_layers no) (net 31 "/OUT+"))
  (pad "2" thru_hole circle (at 0 2.54) (size 1.7 1.7) (drill 1) (layers "*.Cu" "*.Mask") (remove_unused_layers no) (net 30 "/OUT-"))
  (pad "3" thru_hole circle (at 0 5.08) (size 1.7 1.7) (drill 1) (layers "*.Cu" "*.Mask") (remove_unused_layers no) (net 34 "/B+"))
  (pad "4" thru_hole circle (at 0 7.62) (size 1.7 1.7) (drill 1) (layers "*.Cu" "*.Mask") (remove_unused_layers no) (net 35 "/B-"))
  (pad "5" thru_hole circle (at 0 10.16) (size 1.7 1.7) (drill 1) (layers "*.Cu" "*.Mask") (remove_unused_layers no) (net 32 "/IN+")))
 (gr_rect (start 114.3 71.12) (end 220.98 129.54) (stroke (width 0.05) (type default)) (fill no) (layer "Edge.Cuts"))
 (segment (start 196.07 78.74) (end 195.535 78.205) (width 0.2) (layer "F.Cu") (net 3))
 (segment (start 196.07 78.74) (end 200.66 78.74) (width 0.2) (layer "F.Cu") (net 3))
 (segment (start 195.535 78.205) (end 190.5 78.205) (width 0.2) (layer "F.Cu") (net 3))
 (segment (start 134.345 83.545) (end 134.62 83.82) (width 0.2) (layer "F.Cu") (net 3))
 (segment (start 205.25 78.74) (end 200.66 78.74) (width 0.2) (layer "F.Cu") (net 3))
 (segment (start 116.84 83.545) (end 134.345 83.545) (width 0.2) (layer "F.Cu") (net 3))
 (via (at 134.62 83.82) (size 0.6) (drill 0.3) (layers "F.Cu" "B.Cu") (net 3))
 (via (at 190.5 78.205) (size 0.6) (drill 0.3) (layers "F.Cu" "B.Cu") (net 3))
 (segment (start 146.206 87.511) (end 142.24 83.545) (width 0.2) (layer "B.Cu") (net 3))
 (segment (start 156.945 87.42) (end 156.854 87.511) (width 0.2) (layer "B.Cu") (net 3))
 (segment (start 166.16 78.205) (end 156.945 87.42) (width 0.2) (layer "B.Cu") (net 3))
 (segment (start 156.854 87.511) (end 146.206 87.511) (width 0.2) (layer "B.Cu") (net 3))
 (segment (start 134.895 83.545) (end 142.24 83.545) (width 0.2) (layer "B.Cu") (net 3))
 (segment (start 190.5 78.205) (end 166.16 78.205) (width 0.2) (layer "B.Cu") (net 3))
 (segment (start 134.62 83.82) (end 134.895 83.545) (width 0.2) (layer "B.Cu") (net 3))
 (segment (start 152.4 86.36) (end 152.4 91) (width 0.2) (layer "F.Cu") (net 34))
 (segment (start 149.86 83.82) (end 152.4 86.36) (width 0.2) (layer "F.Cu") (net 34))
 (segment (start 152.4 91) (end 166.62 105.22) (width 0.2) (layer "F.Cu") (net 34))
 (segment (start 148.709 87.749) (end 148.709 80.80324) (width 0.2) (layer "F.Cu") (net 32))
 (segment (start 185.4621 83.82) (end 210.82 83.82) (width 0.2) (layer "F.Cu") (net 32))
 (segment (start 152.589646 80.129) (end 154.314646 78.404) (width 0.2) (layer "F.Cu") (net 32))
 (segment (start 210.82 83.82) (end 215.9 88.9) (width 0.2) (layer "F.Cu") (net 32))
 (segment (start 180.0461 78.404) (end 185.4621 83.82) (width 0.2) (layer "F.Cu") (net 32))
 (segment (start 149.38324 80.129) (end 152.589646 80.129) (width 0.2) (layer "F.Cu") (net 32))
 (segment (start 154.314646 78.404) (end 180.0461 78.404) (width 0.2) (layer "F.Cu") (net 32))
 (segment (start 148.709 80.80324) (end 149.38324 80.129) (width 0.2) (layer "F.Cu") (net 32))
 (segment (start 149.86 88.9) (end 148.709 87.749) (width 0.2) (layer "F.Cu") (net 32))
 (segment (start 118.141 112.724) (end 116.84 114.025) (width 0.2) (layer "F.Cu") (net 16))
 (segment (start 118.141 103.264108) (end 118.141 112.724) (width 0.2) (layer "F.Cu") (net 16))
 (segment (start 147.745108 73.66) (end 118.141 103.264108) (width 0.2) (layer "F.Cu") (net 16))
 (segment (start 196.07 73.66) (end 147.745108 73.66) (width 0.2) (layer "F.Cu") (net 16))
 (segment (start 139.239108 115.404) (end 118.001 115.404) (width 0.2) (layer "F.Cu") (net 17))
 (segment (start 142.778892 117.866) (end 141.701108 117.866) (width 0.2) (layer "F.Cu") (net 17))
 (segment (start 141.701108 117.866) (end 139.239108 115.404) (width 0.2) (layer "F.Cu") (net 17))
 (segment (start 143.541 117.103892) (end 142.778892 117.866) (width 0.2) (layer "F.Cu") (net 17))
 (segment (start 118.001 115.404) (end 116.84 116.565) (width 0.2) (layer "F.Cu") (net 17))
 (segment (start 199.271 75.049) (end 151.249 75.049) (width 0.2) (layer "F.Cu") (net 17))
 (segment (start 200.66 73.66) (end 199.271 75.049) (width 0.2) (layer "F.Cu") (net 17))
 (segment (start 143.541 82.757) (end 143.541 117.103892) (width 0.2) (layer "F.Cu") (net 17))
 (segment (start 151.249 75.049) (end 143.541 82.757) (width 0.2) (layer "F.Cu") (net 17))
 (segment (start 203.2 73.66) (end 205.25 73.66) (width 0.2) (layer "F.Cu") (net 1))
 (via (at 203.2 73.66) (size 0.6) (drill 0.3) (layers "F.Cu" "B.Cu") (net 1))
 (segment (start 203.2 73.66) (end 203.2 78.74) (width 0.2) (layer "B.Cu") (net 1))
 (segment (start 203.2 78.74) (end 183.155 98.785) (width 0.2) (layer "B.Cu") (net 1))
 (segment (start 183.155 98.785) (end 142.24 98.785) (width 0.2) (layer "B.Cu") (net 1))
 (segment (start 149.86 81.28) (end 150.616 82.036) (width 0.2) (layer "F.Cu") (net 30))
 (segment (start 183.111 82.036) (end 188.495 87.42) (width 0.2) (layer "F.Cu") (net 30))
 (segment (start 150.616 82.036) (end 183.111 82.036) (width 0.2) (layer "F.Cu") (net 30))
 (segment (start 149.86 86.36) (end 151.999 88.499) (width 0.2) (layer "F.Cu") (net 35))
 (segment (start 151.999 88.499) (end 151.999 103.299) (width 0.2) (layer "F.Cu") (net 35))
 (segment (start 151.999 103.299) (end 166.62 117.92) (width 0.2) (layer "F.Cu") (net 35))
 (segment (start 200.66 76.2) (end 196.07 76.2) (width 0.2) (layer "F.Cu") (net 2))
 (segment (start 196.07 76.2) (end 190.5 76.2) (width 0.2) (layer "F.Cu") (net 2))
 (segment (start 205.25 76.2) (end 200.66 76.2) (width 0.2) (layer "F.Cu") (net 2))
 (via (at 190.5 76.2) (size 0.6) (drill 0.3) (layers "F.Cu" "B.Cu") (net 2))
 (segment (start 160.965 76.2) (end 156.945 80.22) (width 0.2) (layer "B.Cu") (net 2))
 (segment (start 142.24 81.005) (end 143.24 80.005) (width 0.2) (layer "B.Cu") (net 2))
 (segment (start 143.24 80.005) (end 156.73 80.005) (width 0.2) (layer "B.Cu") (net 2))
 (segment (start 190.5 76.2) (end 160.965 76.2) (width 0.2) (layer "B.Cu") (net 2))
 (segment (start 156.73 80.005) (end 156.945 80.22) (width 0.2) (layer "B.Cu") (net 2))
 (segment (start 216.955 90.345) (end 216.955 88.463004) (width 0.2) (layer "F.Cu") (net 31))
 (segment (start 215.9 91.4) (end 216.955 90.345) (width 0.2) (layer "F.Cu") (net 31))
 (segment (start 216.336996 87.845) (end 215.463004 87.845) (width 0.2) (layer "F.Cu") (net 31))
 (segment (start 215.463004 87.845) (end 207.838004 80.22) (width 0.2) (layer "F.Cu") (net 31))
 (segment (start 184.475 76.2) (end 188.495 80.22) (width 0.2) (layer "F.Cu") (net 31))
 (segment (start 152.4 76.2) (end 184.475 76.2) (width 0.2) (layer "F.Cu") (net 31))
 (segment (start 207.838004 80.22) (end 188.495 80.22) (width 0.2) (layer "F.Cu") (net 31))
 (segment (start 149.86 78.74) (end 152.4 76.2) (width 0.2) (layer "F.Cu") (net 31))
 (segment (start 216.955 88.463004) (end 216.336996 87.845) (width 0.2) (layer "F.Cu") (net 31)))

